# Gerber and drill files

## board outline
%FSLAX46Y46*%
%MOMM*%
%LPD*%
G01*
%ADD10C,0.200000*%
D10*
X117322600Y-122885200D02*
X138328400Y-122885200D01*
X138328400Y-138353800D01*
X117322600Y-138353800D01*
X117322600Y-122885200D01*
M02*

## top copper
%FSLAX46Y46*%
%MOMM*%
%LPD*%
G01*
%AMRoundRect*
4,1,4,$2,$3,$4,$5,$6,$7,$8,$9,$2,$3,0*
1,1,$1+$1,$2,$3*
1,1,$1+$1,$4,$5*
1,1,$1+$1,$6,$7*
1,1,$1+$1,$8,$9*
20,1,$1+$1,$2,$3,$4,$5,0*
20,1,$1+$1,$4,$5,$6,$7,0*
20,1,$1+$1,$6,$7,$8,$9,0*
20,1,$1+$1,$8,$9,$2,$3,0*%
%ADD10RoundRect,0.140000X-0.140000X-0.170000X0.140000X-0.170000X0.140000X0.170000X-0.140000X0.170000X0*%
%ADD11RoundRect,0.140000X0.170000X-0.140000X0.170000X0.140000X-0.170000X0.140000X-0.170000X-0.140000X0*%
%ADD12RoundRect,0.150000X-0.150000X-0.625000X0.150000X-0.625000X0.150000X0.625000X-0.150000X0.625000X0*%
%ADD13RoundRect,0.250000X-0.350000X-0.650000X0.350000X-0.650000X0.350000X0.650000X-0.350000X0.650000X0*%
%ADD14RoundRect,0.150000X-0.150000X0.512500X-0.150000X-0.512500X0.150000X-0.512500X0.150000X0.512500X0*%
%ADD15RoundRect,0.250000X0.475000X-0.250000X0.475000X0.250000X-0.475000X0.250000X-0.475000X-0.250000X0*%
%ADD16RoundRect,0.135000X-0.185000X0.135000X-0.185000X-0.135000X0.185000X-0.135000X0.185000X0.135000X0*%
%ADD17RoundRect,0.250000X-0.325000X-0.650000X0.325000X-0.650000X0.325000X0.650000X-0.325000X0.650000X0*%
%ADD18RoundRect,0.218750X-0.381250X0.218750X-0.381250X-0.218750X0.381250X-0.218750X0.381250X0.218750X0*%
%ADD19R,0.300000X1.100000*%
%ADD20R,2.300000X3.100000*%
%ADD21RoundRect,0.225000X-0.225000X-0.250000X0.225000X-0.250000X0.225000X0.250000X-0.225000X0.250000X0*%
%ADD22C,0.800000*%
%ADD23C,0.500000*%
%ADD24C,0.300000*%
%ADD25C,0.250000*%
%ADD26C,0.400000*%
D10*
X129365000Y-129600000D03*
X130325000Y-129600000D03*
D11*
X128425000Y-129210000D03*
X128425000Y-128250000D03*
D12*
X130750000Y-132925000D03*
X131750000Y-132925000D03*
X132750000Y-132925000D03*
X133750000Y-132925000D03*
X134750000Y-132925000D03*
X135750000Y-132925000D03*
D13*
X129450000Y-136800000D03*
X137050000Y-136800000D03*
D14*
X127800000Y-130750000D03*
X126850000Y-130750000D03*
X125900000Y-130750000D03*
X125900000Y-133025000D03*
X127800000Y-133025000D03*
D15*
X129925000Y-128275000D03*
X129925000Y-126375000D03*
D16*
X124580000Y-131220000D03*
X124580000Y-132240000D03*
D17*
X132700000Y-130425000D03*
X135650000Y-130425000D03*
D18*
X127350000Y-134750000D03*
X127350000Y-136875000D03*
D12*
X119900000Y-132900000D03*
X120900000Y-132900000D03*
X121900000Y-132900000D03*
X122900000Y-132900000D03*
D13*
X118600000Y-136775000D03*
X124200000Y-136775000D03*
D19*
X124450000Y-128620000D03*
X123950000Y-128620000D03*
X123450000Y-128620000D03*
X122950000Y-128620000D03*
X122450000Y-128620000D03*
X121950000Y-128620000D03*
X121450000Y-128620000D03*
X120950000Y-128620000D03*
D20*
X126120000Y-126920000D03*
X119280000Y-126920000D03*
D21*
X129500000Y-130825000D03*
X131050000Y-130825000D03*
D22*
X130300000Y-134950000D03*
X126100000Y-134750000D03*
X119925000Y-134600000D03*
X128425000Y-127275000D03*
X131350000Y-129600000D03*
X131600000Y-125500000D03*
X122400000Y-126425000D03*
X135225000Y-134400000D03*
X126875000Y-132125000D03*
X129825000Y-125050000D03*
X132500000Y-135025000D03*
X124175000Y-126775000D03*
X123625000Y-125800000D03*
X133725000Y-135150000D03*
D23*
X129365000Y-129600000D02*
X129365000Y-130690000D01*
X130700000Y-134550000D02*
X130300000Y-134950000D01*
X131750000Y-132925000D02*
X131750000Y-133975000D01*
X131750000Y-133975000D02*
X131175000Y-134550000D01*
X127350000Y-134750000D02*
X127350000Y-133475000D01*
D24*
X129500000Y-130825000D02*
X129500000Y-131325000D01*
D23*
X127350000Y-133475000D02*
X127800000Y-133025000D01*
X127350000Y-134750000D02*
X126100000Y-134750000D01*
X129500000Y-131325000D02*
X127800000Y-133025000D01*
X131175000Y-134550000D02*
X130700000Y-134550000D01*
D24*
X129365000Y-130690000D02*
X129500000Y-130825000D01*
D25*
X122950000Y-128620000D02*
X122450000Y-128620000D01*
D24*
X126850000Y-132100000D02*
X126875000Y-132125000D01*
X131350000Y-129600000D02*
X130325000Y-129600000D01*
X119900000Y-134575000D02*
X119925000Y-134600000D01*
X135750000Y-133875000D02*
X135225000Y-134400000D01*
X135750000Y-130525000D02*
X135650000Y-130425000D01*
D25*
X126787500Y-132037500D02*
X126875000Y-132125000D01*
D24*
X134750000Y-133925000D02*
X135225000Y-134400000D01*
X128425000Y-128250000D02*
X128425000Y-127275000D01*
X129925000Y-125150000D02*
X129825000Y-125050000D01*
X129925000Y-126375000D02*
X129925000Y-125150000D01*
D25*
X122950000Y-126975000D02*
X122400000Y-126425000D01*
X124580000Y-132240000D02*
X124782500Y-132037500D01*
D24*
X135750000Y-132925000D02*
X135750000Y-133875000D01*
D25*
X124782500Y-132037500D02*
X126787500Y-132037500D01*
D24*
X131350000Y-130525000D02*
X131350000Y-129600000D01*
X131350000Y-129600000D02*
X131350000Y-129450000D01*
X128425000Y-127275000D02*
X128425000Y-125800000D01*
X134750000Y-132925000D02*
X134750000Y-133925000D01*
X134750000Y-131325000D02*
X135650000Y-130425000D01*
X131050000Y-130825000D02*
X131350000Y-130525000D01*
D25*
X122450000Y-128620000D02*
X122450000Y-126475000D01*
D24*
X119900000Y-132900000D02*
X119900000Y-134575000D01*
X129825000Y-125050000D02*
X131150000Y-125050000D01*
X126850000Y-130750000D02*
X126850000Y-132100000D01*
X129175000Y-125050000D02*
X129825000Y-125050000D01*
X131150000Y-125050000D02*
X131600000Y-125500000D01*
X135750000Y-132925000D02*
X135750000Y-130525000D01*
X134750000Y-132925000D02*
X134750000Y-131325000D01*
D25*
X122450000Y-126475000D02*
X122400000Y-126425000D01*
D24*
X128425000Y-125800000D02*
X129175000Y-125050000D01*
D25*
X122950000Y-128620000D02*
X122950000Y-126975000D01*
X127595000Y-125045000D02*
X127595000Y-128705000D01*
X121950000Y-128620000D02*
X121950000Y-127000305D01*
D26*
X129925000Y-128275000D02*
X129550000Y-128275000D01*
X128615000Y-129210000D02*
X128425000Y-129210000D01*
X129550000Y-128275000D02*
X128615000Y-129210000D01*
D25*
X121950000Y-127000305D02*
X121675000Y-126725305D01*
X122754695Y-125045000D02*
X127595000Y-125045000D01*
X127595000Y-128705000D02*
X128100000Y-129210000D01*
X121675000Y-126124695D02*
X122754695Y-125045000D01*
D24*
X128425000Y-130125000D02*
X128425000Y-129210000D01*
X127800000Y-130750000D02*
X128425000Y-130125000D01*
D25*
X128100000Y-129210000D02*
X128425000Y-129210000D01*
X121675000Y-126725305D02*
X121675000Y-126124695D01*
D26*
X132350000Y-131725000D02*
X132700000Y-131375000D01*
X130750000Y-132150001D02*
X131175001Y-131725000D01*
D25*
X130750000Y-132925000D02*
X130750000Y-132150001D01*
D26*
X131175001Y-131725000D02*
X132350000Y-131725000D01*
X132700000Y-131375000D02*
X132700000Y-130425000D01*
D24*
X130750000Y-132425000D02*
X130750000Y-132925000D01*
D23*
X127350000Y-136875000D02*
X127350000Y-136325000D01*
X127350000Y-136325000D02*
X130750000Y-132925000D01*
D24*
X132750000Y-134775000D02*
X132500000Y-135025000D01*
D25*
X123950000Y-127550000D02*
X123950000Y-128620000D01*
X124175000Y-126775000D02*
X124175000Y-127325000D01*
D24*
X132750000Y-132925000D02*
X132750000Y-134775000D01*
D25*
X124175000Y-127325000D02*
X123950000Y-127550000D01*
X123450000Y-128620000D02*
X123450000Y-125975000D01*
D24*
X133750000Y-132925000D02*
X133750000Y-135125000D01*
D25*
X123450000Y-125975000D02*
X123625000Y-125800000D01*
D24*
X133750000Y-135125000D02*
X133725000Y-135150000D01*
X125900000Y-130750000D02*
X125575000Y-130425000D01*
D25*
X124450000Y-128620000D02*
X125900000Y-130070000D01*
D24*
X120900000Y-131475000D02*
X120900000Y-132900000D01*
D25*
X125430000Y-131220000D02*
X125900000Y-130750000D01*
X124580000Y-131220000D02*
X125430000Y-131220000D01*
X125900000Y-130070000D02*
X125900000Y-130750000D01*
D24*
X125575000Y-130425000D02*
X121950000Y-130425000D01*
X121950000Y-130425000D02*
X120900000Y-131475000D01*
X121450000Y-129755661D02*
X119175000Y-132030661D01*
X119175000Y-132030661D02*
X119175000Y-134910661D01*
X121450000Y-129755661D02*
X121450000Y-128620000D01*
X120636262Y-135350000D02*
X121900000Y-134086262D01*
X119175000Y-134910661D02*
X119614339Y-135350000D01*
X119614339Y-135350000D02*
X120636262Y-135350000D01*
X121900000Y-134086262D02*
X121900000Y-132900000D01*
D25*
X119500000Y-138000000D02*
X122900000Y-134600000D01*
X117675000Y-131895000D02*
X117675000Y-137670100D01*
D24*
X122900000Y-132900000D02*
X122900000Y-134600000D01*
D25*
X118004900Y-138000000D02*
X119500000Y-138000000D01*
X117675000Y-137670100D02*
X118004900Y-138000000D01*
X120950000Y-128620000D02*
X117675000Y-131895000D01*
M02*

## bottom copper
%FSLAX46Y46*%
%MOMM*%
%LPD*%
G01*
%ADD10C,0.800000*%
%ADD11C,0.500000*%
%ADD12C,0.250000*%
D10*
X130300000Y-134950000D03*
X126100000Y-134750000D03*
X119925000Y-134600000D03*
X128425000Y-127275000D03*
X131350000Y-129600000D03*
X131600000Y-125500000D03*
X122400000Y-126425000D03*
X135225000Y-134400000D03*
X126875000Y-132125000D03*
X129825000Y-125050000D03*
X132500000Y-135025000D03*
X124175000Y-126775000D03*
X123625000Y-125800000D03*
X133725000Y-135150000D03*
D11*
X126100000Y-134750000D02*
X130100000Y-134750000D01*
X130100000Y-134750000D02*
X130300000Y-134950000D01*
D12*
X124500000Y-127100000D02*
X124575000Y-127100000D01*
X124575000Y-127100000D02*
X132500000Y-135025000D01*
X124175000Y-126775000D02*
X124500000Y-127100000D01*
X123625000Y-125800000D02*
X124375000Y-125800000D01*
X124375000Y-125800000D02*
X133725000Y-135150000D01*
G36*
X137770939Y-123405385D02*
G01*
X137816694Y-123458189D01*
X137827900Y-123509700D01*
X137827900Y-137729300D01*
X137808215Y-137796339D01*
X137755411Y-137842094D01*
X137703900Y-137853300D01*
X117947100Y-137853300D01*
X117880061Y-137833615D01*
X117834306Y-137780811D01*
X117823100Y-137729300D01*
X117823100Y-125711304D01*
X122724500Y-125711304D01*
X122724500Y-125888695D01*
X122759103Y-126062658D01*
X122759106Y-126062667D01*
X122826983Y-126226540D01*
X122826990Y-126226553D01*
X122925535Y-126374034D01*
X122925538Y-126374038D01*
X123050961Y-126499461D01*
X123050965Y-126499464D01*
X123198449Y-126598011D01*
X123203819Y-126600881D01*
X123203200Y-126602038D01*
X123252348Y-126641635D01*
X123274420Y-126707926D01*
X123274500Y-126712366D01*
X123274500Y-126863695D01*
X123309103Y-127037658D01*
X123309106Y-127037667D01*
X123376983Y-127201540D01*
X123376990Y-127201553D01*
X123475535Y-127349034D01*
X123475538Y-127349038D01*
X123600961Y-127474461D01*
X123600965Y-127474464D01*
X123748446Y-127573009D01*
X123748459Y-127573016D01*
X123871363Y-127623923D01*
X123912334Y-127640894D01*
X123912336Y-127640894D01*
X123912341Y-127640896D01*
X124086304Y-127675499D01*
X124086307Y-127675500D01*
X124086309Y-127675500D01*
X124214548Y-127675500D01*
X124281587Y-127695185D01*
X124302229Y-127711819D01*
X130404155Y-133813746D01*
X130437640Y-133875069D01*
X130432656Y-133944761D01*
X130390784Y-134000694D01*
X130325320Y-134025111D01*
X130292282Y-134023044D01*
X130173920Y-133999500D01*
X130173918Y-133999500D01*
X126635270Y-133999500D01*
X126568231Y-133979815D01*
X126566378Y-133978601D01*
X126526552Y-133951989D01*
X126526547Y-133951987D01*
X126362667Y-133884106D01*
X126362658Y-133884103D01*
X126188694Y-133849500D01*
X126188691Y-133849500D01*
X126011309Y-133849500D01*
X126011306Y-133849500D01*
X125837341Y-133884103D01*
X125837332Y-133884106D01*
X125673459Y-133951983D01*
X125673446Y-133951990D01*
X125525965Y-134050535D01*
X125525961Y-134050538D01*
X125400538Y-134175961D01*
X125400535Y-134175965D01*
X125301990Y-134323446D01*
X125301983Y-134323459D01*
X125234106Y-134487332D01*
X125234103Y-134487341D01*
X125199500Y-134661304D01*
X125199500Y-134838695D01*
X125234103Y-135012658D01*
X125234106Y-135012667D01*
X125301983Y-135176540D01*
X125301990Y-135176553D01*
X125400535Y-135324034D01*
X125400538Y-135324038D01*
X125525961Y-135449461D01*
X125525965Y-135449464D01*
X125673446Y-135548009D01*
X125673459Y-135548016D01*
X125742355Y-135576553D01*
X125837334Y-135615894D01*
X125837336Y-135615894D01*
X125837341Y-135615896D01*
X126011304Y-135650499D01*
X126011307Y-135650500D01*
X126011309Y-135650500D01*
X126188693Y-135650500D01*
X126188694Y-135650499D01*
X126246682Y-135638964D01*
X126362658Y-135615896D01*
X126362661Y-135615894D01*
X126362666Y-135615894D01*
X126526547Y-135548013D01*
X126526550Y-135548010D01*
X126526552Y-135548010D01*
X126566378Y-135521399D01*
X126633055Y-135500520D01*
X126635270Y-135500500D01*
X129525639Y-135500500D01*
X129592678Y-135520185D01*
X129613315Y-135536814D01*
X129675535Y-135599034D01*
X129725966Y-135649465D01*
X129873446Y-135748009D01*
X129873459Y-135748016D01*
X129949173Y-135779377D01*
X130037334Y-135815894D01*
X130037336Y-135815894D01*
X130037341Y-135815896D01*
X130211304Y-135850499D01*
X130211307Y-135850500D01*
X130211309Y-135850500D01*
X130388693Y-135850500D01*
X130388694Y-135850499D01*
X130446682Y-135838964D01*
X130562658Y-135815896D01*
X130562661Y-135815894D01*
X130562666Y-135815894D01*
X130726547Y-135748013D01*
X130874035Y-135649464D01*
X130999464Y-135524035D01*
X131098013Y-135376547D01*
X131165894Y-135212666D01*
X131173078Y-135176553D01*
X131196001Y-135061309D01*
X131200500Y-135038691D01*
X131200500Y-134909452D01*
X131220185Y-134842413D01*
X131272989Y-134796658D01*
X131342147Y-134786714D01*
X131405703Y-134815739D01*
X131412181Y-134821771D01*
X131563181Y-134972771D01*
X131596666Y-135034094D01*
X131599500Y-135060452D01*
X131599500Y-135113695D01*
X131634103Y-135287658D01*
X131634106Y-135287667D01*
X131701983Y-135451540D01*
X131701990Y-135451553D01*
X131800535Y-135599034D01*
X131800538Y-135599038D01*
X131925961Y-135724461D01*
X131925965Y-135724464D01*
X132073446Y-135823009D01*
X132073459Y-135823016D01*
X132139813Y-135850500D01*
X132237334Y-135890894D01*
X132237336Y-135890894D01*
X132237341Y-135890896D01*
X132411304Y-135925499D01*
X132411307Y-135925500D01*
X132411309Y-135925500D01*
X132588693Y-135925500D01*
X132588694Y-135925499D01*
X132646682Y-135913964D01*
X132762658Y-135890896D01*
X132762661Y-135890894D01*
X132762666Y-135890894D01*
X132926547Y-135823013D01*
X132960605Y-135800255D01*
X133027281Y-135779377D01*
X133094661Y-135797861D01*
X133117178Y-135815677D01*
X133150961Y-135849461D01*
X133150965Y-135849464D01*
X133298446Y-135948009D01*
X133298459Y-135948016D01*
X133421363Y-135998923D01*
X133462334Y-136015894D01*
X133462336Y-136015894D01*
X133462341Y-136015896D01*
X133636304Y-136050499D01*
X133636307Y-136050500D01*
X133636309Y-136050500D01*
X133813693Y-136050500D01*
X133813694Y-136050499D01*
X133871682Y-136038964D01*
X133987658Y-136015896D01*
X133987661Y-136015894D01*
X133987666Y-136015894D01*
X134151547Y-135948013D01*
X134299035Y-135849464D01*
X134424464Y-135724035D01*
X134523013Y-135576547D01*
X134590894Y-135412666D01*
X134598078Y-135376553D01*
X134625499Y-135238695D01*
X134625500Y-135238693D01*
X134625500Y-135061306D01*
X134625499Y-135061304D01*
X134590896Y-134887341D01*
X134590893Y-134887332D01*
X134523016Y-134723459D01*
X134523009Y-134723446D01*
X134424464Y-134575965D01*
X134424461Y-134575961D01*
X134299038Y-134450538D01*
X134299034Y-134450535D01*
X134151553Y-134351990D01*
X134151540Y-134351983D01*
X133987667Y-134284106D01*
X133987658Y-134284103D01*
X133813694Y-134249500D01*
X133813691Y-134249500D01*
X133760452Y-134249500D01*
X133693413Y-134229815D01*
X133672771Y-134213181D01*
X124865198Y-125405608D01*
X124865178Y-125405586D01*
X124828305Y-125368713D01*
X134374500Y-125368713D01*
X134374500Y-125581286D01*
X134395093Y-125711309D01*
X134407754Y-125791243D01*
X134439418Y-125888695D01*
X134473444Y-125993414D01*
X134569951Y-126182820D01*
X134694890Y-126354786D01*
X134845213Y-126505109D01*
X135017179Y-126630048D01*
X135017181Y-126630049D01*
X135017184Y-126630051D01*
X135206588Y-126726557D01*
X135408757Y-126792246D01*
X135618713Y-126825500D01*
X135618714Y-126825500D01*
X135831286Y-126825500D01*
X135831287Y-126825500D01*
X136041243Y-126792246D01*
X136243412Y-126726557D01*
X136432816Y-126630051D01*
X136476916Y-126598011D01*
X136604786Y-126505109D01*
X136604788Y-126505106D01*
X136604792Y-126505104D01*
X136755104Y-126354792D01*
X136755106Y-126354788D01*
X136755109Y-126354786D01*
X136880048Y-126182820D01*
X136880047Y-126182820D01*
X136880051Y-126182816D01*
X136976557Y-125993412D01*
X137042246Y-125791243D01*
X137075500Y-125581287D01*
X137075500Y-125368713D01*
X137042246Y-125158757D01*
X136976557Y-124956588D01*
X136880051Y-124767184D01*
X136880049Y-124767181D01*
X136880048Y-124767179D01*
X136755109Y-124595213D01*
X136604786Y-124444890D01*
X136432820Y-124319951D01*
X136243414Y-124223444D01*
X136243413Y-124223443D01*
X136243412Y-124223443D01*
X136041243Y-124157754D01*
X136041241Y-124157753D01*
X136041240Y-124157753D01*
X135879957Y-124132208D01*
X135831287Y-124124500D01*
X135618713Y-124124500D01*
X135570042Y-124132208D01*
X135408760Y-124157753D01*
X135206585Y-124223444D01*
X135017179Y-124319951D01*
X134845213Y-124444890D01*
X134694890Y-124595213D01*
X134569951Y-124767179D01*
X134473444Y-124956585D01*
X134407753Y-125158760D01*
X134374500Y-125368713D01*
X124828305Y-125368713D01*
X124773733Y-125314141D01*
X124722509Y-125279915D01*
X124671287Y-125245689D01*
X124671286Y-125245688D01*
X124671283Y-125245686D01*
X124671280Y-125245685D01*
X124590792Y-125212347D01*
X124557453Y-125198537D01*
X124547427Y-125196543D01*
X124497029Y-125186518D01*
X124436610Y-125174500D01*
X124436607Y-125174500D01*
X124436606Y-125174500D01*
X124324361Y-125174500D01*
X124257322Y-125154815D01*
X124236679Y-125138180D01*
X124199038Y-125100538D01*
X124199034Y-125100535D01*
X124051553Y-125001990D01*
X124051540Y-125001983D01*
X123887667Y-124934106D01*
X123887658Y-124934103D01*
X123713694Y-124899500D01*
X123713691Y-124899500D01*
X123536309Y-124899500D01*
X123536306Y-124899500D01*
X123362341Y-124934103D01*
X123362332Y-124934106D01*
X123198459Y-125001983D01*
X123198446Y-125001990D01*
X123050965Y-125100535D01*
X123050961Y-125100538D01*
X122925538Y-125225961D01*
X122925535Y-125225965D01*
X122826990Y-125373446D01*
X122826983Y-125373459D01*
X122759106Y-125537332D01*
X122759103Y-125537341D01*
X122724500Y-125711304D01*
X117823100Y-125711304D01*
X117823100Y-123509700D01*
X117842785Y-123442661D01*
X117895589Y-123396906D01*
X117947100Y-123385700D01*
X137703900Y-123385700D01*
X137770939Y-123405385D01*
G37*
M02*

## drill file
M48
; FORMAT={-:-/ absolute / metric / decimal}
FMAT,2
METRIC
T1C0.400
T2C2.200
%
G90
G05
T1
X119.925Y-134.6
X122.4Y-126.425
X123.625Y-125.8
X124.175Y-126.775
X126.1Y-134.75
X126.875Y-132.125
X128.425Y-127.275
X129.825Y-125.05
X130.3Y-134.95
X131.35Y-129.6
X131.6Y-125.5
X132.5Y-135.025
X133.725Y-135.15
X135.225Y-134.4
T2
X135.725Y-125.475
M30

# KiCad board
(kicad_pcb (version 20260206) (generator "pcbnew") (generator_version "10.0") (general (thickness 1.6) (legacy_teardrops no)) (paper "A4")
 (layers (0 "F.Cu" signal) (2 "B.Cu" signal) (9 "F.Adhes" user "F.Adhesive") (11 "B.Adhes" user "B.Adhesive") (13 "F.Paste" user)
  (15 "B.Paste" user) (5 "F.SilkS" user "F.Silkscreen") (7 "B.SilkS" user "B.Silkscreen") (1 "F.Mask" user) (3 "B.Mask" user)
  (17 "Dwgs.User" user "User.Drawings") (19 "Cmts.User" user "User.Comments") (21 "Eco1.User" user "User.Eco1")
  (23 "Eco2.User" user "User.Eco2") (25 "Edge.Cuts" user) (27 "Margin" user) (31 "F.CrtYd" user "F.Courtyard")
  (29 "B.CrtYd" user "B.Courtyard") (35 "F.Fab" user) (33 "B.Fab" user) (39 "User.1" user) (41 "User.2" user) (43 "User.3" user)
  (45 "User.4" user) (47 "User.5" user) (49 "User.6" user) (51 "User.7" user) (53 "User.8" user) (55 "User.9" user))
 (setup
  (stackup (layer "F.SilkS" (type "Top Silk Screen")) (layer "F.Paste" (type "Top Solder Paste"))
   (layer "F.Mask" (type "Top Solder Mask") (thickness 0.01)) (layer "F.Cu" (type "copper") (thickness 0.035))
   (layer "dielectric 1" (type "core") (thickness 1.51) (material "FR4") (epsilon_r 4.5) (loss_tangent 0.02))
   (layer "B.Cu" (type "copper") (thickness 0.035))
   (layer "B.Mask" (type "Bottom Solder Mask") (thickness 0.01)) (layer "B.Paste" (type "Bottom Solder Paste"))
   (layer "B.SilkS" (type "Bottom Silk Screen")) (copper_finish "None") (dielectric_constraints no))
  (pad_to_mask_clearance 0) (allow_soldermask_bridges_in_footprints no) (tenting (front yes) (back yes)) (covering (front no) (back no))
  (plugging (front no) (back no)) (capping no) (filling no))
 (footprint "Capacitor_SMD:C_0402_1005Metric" (layer "F.Cu") (at 129.845 129.6)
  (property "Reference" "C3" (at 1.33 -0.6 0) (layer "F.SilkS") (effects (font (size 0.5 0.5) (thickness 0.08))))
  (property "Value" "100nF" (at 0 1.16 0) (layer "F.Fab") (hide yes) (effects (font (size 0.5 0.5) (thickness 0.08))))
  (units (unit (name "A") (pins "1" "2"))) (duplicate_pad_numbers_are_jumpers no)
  (pad "1" smd roundrect (at -0.48 0) (size 0.56 0.62) (layers "F.Cu" "F.Mask" "F.Paste") (roundrect_rratio 0.25) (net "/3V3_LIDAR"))
  (pad "2" smd roundrect (at 0.48 0) (size 0.56 0.62) (layers "F.Cu" "F.Mask" "F.Paste") (roundrect_rratio 0.25) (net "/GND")))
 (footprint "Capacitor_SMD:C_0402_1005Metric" (layer "F.Cu") (at 128.425 128.73 90)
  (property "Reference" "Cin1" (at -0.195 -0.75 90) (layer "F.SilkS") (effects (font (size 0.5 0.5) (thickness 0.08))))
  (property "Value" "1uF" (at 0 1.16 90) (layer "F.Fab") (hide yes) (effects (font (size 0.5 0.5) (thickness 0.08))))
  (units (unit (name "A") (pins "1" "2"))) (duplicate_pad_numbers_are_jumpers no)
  (pad "1" smd roundrect (at -0.48 0 90) (size 0.56 0.62) (layers "F.Cu" "F.Mask" "F.Paste") (roundrect_rratio 0.25) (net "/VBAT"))
  (pad "2" smd roundrect (at 0.48 0 90) (size 0.56 0.62) (layers "F.Cu" "F.Mask" "F.Paste") (roundrect_rratio 0.25) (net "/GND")))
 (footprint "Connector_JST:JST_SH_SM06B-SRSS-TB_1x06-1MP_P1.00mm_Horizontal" (layer "F.Cu") (at 133.25 134.925)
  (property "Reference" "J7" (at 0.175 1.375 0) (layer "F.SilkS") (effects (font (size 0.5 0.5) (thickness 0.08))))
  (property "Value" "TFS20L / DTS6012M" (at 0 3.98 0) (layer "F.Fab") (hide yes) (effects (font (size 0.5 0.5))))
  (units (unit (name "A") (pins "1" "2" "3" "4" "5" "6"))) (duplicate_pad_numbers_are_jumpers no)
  (pad "1" smd roundrect (at -2.5 -2) (size 0.6 1.55) (layers "F.Cu" "F.Mask" "F.Paste") (roundrect_rratio 0.25) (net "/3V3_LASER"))
  (pad "2" smd roundrect (at -1.5 -2) (size 0.6 1.55) (layers "F.Cu" "F.Mask" "F.Paste") (roundrect_rratio 0.25) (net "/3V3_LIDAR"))
  (pad "3" smd roundrect (at -0.5 -2) (size 0.6 1.55) (layers "F.Cu" "F.Mask" "F.Paste") (roundrect_rratio 0.25) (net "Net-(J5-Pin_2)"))
  (pad "4" smd roundrect (at 0.5 -2) (size 0.6 1.55) (layers "F.Cu" "F.Mask" "F.Paste") (roundrect_rratio 0.25) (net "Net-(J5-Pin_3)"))
  (pad "5" smd roundrect (at 1.5 -2) (size 0.6 1.55) (layers "F.Cu" "F.Mask" "F.Paste") (roundrect_rratio 0.25) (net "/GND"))
  (pad "6" smd roundrect (at 2.5 -2) (size 0.6 1.55) (layers "F.Cu" "F.Mask" "F.Paste") (roundrect_rratio 0.25) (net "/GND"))
  (pad "MP" smd roundrect (at -3.8 1.875) (size 1.2 1.8) (layers "F.Cu" "F.Mask" "F.Paste") (roundrect_rratio 0.208333))
  (pad "MP" smd roundrect (at 3.8 1.875) (size 1.2 1.8) (layers "F.Cu" "F.Mask" "F.Paste") (roundrect_rratio 0.208333)))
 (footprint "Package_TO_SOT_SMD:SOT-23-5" (layer "F.Cu") (at 126.85 131.8875 -90)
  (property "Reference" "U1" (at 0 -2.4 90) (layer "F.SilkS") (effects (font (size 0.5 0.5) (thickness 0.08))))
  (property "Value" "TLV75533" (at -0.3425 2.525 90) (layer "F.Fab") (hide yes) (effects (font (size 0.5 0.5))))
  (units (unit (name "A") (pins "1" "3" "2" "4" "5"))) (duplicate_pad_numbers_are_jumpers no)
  (pad "1" smd roundrect (at -1.1375 -0.95 270) (size 1.325 0.6) (layers "F.Cu" "F.Mask" "F.Paste") (roundrect_rratio 0.25) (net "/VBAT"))
  (pad "2" smd roundrect (at -1.1375 0 270) (size 1.325 0.6) (layers "F.Cu" "F.Mask" "F.Paste") (roundrect_rratio 0.25) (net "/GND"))
  (pad "3" smd roundrect (at -1.1375 0.95 270) (size 1.325 0.6) (layers "F.Cu" "F.Mask" "F.Paste") (roundrect_rratio 0.25) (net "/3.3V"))
  (pad "4" smd roundrect (at 1.1375 0.95 270) (size 1.325 0.6) (layers "F.Cu" "F.Mask" "F.Paste") (roundrect_rratio 0.25)
   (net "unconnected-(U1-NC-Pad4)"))
  (pad "5" smd roundrect (at 1.1375 -0.95 270) (size 1.325 0.6) (layers "F.Cu" "F.Mask" "F.Paste") (roundrect_rratio 0.25)
   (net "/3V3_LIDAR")))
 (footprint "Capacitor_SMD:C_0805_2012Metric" (layer "F.Cu") (at 129.925 127.325 90)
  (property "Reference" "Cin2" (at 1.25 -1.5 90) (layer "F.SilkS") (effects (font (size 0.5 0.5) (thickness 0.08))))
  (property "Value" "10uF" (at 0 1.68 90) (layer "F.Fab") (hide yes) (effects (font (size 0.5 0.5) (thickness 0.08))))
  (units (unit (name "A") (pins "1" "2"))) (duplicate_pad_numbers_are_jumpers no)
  (pad "1" smd roundrect (at -0.95 0 90) (size 1 1.45) (layers "F.Cu" "F.Mask" "F.Paste") (roundrect_rratio 0.25) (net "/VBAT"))
  (pad "2" smd roundrect (at 0.95 0 90) (size 1 1.45) (layers "F.Cu" "F.Mask" "F.Paste") (roundrect_rratio 0.25) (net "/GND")))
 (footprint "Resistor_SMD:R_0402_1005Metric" (layer "F.Cu") (at 124.58 131.73 -90)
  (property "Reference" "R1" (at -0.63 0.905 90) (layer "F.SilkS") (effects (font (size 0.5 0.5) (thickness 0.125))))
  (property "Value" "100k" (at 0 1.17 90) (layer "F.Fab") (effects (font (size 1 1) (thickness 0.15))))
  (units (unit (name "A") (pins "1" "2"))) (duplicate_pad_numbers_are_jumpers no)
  (pad "1" smd roundrect (at -0.51 0 270) (size 0.54 0.64) (layers "F.Cu" "F.Mask" "F.Paste") (roundrect_rratio 0.25) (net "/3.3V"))
  (pad "2" smd roundrect (at 0.51 0 270) (size 0.54 0.64) (layers "F.Cu" "F.Mask" "F.Paste") (roundrect_rratio 0.25) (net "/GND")))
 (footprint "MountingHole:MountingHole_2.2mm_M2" (layer "F.Cu") (at 135.725 125.475)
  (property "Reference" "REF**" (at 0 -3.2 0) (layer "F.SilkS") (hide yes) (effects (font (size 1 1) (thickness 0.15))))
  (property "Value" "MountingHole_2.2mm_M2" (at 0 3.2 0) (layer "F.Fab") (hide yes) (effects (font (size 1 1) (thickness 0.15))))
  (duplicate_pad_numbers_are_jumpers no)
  (pad "" np_thru_hole circle (at 0 0) (size 2.2 2.2) (drill 2.2) (layers "*.Cu" "*.Mask")))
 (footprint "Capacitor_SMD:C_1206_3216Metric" (layer "F.Cu") (at 134.175 130.425)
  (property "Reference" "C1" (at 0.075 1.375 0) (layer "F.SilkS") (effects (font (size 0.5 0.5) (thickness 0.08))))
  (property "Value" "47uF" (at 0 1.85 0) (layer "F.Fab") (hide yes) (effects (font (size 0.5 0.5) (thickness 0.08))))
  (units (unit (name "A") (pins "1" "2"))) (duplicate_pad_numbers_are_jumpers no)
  (pad "1" smd roundrect (at -1.475 0) (size 1.15 1.8) (layers "F.Cu" "F.Mask" "F.Paste") (roundrect_rratio 0.217391) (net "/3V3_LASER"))
  (pad "2" smd roundrect (at 1.475 0) (size 1.15 1.8) (layers "F.Cu" "F.Mask" "F.Paste") (roundrect_rratio 0.217391) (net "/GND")))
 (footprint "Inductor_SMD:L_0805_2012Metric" (layer "F.Cu") (at 127.35 135.8125 -90)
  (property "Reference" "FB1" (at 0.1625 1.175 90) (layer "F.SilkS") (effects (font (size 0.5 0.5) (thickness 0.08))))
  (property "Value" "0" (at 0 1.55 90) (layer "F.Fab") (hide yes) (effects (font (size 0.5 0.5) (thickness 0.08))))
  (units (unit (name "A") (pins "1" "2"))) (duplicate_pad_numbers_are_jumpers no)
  (pad "1" smd roundrect (at -1.0625 0 270) (size 0.875 1.2) (layers "F.Cu" "F.Mask" "F.Paste") (roundrect_rratio 0.25) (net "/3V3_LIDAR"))
  (pad "2" smd roundrect (at 1.0625 0 270) (size 0.875 1.2) (layers "F.Cu" "F.Mask" "F.Paste") (roundrect_rratio 0.25) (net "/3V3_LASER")))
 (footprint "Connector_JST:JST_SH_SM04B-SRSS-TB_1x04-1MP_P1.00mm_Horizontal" (layer "F.Cu") (at 121.4 134.9)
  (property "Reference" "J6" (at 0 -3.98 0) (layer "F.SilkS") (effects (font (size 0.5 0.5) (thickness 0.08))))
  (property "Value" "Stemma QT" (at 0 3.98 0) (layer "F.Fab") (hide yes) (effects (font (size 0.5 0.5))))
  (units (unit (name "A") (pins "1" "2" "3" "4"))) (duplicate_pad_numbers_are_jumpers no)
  (pad "1" smd roundrect (at -1.5 -2) (size 0.6 1.55) (layers "F.Cu" "F.Mask" "F.Paste") (roundrect_rratio 0.25) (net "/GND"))
  (pad "2" smd roundrect (at -0.5 -2) (size 0.6 1.55) (layers "F.Cu" "F.Mask" "F.Paste") (roundrect_rratio 0.25) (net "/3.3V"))
  (pad "3" smd roundrect (at 0.5 -2) (size 0.6 1.55) (layers "F.Cu" "F.Mask" "F.Paste") (roundrect_rratio 0.25) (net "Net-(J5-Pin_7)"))
  (pad "4" smd roundrect (at 1.5 -2) (size 0.6 1.55) (layers "F.Cu" "F.Mask" "F.Paste") (roundrect_rratio 0.25) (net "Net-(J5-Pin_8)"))
  (pad "MP" smd roundrect (at -2.8 1.875) (size 1.2 1.8) (layers "F.Cu" "F.Mask" "F.Paste") (roundrect_rratio 0.208333))
  (pad "MP" smd roundrect (at 2.8 1.875) (size 1.2 1.8) (layers "F.Cu" "F.Mask" "F.Paste") (roundrect_rratio 0.208333)))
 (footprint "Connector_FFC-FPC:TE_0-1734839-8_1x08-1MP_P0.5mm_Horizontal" (layer "F.Cu") (at 122.7 127.27 180)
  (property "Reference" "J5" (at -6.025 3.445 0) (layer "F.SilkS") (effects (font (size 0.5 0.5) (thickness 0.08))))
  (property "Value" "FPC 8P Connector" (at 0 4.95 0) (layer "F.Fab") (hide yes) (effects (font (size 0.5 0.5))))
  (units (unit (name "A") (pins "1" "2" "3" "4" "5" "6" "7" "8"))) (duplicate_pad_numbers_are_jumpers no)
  (pad "1" smd rect (at -1.75 -1.35 180) (size 0.3 1.1) (layers "F.Cu" "F.Mask" "F.Paste") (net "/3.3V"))
  (pad "2" smd rect (at -1.25 -1.35 180) (size 0.3 1.1) (layers "F.Cu" "F.Mask" "F.Paste") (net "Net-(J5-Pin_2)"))
  (pad "3" smd rect (at -0.75 -1.35 180) (size 0.3 1.1) (layers "F.Cu" "F.Mask" "F.Paste") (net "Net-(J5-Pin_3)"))
  (pad "4" smd rect (at -0.25 -1.35 180) (size 0.3 1.1) (layers "F.Cu" "F.Mask" "F.Paste") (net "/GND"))
  (pad "5" smd rect (at 0.25 -1.35 180) (size 0.3 1.1) (layers "F.Cu" "F.Mask" "F.Paste") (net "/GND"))
  (pad "6" smd rect (at 0.75 -1.35 180) (size 0.3 1.1) (layers "F.Cu" "F.Mask" "F.Paste") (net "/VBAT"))
  (pad "7" smd rect (at 1.25 -1.35 180) (size 0.3 1.1) (layers "F.Cu" "F.Mask" "F.Paste") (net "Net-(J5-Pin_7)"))
  (pad "8" smd rect (at 1.75 -1.35 180) (size 0.3 1.1) (layers "F.Cu" "F.Mask" "F.Paste") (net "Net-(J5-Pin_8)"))
  (pad "MP" smd rect (at -3.42 0.35 180) (size 2.3 3.1) (layers "F.Cu" "F.Mask" "F.Paste"))
  (pad "MP" smd rect (at 3.42 0.35 180) (size 2.3 3.1) (layers "F.Cu" "F.Mask" "F.Paste")))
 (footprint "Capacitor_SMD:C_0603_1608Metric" (layer "F.Cu") (at 130.275 130.825)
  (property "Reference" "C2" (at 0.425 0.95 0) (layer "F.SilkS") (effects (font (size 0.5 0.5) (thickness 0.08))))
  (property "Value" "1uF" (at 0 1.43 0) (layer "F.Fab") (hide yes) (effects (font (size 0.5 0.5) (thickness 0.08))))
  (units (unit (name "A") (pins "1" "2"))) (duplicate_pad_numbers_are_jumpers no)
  (pad "1" smd roundrect (at -0.775 0) (size 0.9 0.95) (layers "F.Cu" "F.Mask" "F.Paste") (roundrect_rratio 0.25) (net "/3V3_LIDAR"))
  (pad "2" smd roundrect (at 0.775 0) (size 0.9 0.95) (layers "F.Cu" "F.Mask" "F.Paste") (roundrect_rratio 0.25) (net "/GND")))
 (gr_rect (start 117.3226 122.8852) (end 138.3284 138.3538) (stroke (width 0.2) (type default)) (fill no) (layer "Edge.Cuts"))
 (segment (start 129.365 129.6) (end 129.365 130.69) (width 0.5) (layer "F.Cu") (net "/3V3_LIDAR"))
 (segment (start 130.7 134.55) (end 130.3 134.95) (width 0.5) (layer "F.Cu") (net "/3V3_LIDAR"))
 (segment (start 131.75 132.925) (end 131.75 133.975) (width 0.5) (layer "F.Cu") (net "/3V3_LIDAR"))
 (segment (start 131.75 133.975) (end 131.175 134.55) (width 0.5) (layer "F.Cu") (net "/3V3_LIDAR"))
 (segment (start 127.35 134.75) (end 127.35 133.475) (width 0.5) (layer "F.Cu") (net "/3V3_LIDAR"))
 (segment (start 129.5 130.825) (end 129.5 131.325) (width 0.3) (layer "F.Cu") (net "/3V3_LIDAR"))
 (segment (start 127.35 133.475) (end 127.8 133.025) (width 0.5) (layer "F.Cu") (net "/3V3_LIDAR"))
 (segment (start 127.35 134.75) (end 126.1 134.75) (width 0.5) (layer "F.Cu") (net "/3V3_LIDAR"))
 (segment (start 129.5 131.325) (end 127.8 133.025) (width 0.5) (layer "F.Cu") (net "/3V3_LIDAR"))
 (segment (start 131.175 134.55) (end 130.7 134.55) (width 0.5) (layer "F.Cu") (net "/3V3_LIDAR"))
 (segment (start 129.365 130.69) (end 129.5 130.825) (width 0.3) (layer "F.Cu") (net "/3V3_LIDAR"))
 (via (at 130.3 134.95) (size 0.8) (drill 0.4) (layers "F.Cu" "B.Cu") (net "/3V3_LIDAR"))
 (via (at 126.1 134.75) (size 0.8) (drill 0.4) (layers "F.Cu" "B.Cu") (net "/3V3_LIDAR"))
 (segment (start 126.1 134.75) (end 130.1 134.75) (width 0.5) (layer "B.Cu") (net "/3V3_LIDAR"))
 (segment (start 130.1 134.75) (end 130.3 134.95) (width 0.5) (layer "B.Cu") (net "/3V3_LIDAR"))
 (segment (start 122.95 128.62) (end 122.45 128.62) (width 0.25) (layer "F.Cu") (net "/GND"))
 (segment (start 126.85 132.1) (end 126.875 132.125) (width 0.3) (layer "F.Cu") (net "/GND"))
 (segment (start 131.35 129.6) (end 130.325 129.6) (width 0.3) (layer "F.Cu") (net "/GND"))
 (segment (start 119.9 134.575) (end 119.925 134.6) (width 0.3) (layer "F.Cu") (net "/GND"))
 (segment (start 135.75 133.875) (end 135.225 134.4) (width 0.3) (layer "F.Cu") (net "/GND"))
 (segment (start 135.75 130.525) (end 135.65 130.425) (width 0.3) (layer "F.Cu") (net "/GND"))
 (segment (start 126.7875 132.0375) (end 126.875 132.125) (width 0.25) (layer "F.Cu") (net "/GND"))
 (segment (start 134.75 133.925) (end 135.225 134.4) (width 0.3) (layer "F.Cu") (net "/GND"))
 (segment (start 128.425 128.25) (end 128.425 127.275) (width 0.3) (layer "F.Cu") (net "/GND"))
 (segment (start 129.925 125.15) (end 129.825 125.05) (width 0.3) (layer "F.Cu") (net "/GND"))
 (segment (start 129.925 126.375) (end 129.925 125.15) (width 0.3) (layer "F.Cu") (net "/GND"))
 (segment (start 122.95 126.975) (end 122.4 126.425) (width 0.25) (layer "F.Cu") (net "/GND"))
 (segment (start 124.58 132.24) (end 124.7825 132.0375) (width 0.25) (layer "F.Cu") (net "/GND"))
 (segment (start 135.75 132.925) (end 135.75 133.875) (width 0.3) (layer "F.Cu") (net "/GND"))
 (segment (start 124.7825 132.0375) (end 126.7875 132.0375) (width 0.25) (layer "F.Cu") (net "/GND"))
 (segment (start 131.35 130.525) (end 131.35 129.6) (width 0.3) (layer "F.Cu") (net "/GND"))
 (segment (start 131.35 129.6) (end 131.35 129.45) (width 0.3) (layer "F.Cu") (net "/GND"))
 (segment (start 128.425 127.275) (end 128.425 125.8) (width 0.3) (layer "F.Cu") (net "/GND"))
 (segment (start 134.75 132.925) (end 134.75 133.925) (width 0.3) (layer "F.Cu") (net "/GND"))
 (segment (start 134.75 131.325) (end 135.65 130.425) (width 0.3) (layer "F.Cu") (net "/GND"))
 (segment (start 131.05 130.825) (end 131.35 130.525) (width 0.3) (layer "F.Cu") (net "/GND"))
 (segment (start 122.45 128.62) (end 122.45 126.475) (width 0.25) (layer "F.Cu") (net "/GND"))
 (segment (start 119.9 132.9) (end 119.9 134.575) (width 0.3) (layer "F.Cu") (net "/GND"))
 (segment (start 129.825 125.05) (end 131.15 125.05) (width 0.3) (layer "F.Cu") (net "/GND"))
 (segment (start 126.85 130.75) (end 126.85 132.1) (width 0.3) (layer "F.Cu") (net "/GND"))
 (segment (start 129.175 125.05) (end 129.825 125.05) (width 0.3) (layer "F.Cu") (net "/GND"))
 (segment (start 131.15 125.05) (end 131.6 125.5) (width 0.3) (layer "F.Cu") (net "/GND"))
 (segment (start 135.75 132.925) (end 135.75 130.525) (width 0.3) (layer "F.Cu") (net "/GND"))
 (segment (start 134.75 132.925) (end 134.75 131.325) (width 0.3) (layer "F.Cu") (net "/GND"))
 (segment (start 122.45 126.475) (end 122.4 126.425) (width 0.25) (layer "F.Cu") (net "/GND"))
 (segment (start 128.425 125.8) (end 129.175 125.05) (width 0.3) (layer "F.Cu") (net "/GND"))
 (segment (start 122.95 128.62) (end 122.95 126.975) (width 0.25) (layer "F.Cu") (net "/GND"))
 (via (at 119.925 134.6) (size 0.8) (drill 0.4) (layers "F.Cu" "B.Cu") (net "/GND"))
 (via (at 128.425 127.275) (size 0.8) (drill 0.4) (layers "F.Cu" "B.Cu") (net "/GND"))
 (via (at 131.35 129.6) (size 0.8) (drill 0.4) (layers "F.Cu" "B.Cu") (free yes) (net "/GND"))
 (via (at 131.6 125.5) (size 0.8) (drill 0.4) (layers "F.Cu" "B.Cu") (free yes) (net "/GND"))
 (via (at 122.4 126.425) (size 0.8) (drill 0.4) (layers "F.Cu" "B.Cu") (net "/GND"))
 (via (at 135.225 134.4) (size 0.8) (drill 0.4) (layers "F.Cu" "B.Cu") (free yes) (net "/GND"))
 (via (at 126.875 132.125) (size 0.8) (drill 0.4) (layers "F.Cu" "B.Cu") (free yes) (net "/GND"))
 (via (at 129.825 125.05) (size 0.8) (drill 0.4) (layers "F.Cu" "B.Cu") (free yes) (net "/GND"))
 (segment (start 127.595 125.045) (end 127.595 128.705) (width 0.25) (layer "F.Cu") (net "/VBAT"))
 (segment (start 121.95 128.62) (end 121.95 127.000305) (width 0.25) (layer "F.Cu") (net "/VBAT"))
 (segment (start 129.925 128.275) (end 129.55 128.275) (width 0.4) (layer "F.Cu") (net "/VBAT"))
 (segment (start 128.615 129.21) (end 128.425 129.21) (width 0.4) (layer "F.Cu") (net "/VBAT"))
 (segment (start 129.55 128.275) (end 128.615 129.21) (width 0.4) (layer "F.Cu") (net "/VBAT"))
 (segment (start 121.95 127.000305) (end 121.675 126.725305) (width 0.25) (layer "F.Cu") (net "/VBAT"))
 (segment (start 122.754695 125.045) (end 127.595 125.045) (width 0.25) (layer "F.Cu") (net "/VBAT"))
 (segment (start 127.595 128.705) (end 128.1 129.21) (width 0.25) (layer "F.Cu") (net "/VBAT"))
 (segment (start 121.675 126.124695) (end 122.754695 125.045) (width 0.25) (layer "F.Cu") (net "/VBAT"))
 (segment (start 128.425 130.125) (end 128.425 129.21) (width 0.3) (layer "F.Cu") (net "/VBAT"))
 (segment (start 127.8 130.75) (end 128.425 130.125) (width 0.3) (layer "F.Cu") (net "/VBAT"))
 (segment (start 128.1 129.21) (end 128.425 129.21) (width 0.25) (layer "F.Cu") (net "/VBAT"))
 (segment (start 121.675 126.725305) (end 121.675 126.124695) (width 0.25) (layer "F.Cu") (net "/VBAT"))
 (segment (start 132.35 131.725) (end 132.7 131.375) (width 0.4) (layer "F.Cu") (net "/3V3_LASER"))
 (segment (start 130.75 132.150001) (end 131.175001 131.725) (width 0.4) (layer "F.Cu") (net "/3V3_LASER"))
 (segment (start 130.75 132.925) (end 130.75 132.150001) (width 0.25) (layer "F.Cu") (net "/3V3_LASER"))
 (segment (start 131.175001 131.725) (end 132.35 131.725) (width 0.4) (layer "F.Cu") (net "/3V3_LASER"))
 (segment (start 132.7 131.375) (end 132.7 130.425) (width 0.4) (layer "F.Cu") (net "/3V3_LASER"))
 (segment (start 130.75 132.425) (end 130.75 132.925) (width 0.3) (layer "F.Cu") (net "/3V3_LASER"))
 (segment (start 127.35 136.875) (end 127.35 136.325) (width 0.5) (layer "F.Cu") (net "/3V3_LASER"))
 (segment (start 127.35 136.325) (end 130.75 132.925) (width 0.5) (layer "F.Cu") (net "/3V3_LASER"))
 (segment (start 132.75 134.775) (end 132.5 135.025) (width 0.3) (layer "F.Cu") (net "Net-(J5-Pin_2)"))
 (segment (start 123.95 127.55) (end 123.95 128.62) (width 0.25) (layer "F.Cu") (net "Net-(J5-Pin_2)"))
 (segment (start 124.175 126.775) (end 124.175 127.325) (width 0.25) (layer "F.Cu") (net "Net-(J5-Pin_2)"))
 (segment (start 132.75 132.925) (end 132.75 134.775) (width 0.3) (layer "F.Cu") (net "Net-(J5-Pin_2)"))
 (segment (start 124.175 127.325) (end 123.95 127.55) (width 0.25) (layer "F.Cu") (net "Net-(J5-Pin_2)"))
 (via (at 132.5 135.025) (size 0.8) (drill 0.4) (layers "F.Cu" "B.Cu") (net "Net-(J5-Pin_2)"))
 (via (at 124.175 126.775) (size 0.8) (drill 0.4) (layers "F.Cu" "B.Cu") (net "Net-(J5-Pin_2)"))
 (segment (start 124.5 127.1) (end 124.575 127.1) (width 0.25) (layer "B.Cu") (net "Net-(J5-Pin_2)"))
 (segment (start 124.575 127.1) (end 132.5 135.025) (width 0.25) (layer "B.Cu") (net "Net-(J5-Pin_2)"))
 (segment (start 124.175 126.775) (end 124.5 127.1) (width 0.25) (layer "B.Cu") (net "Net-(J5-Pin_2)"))
 (segment (start 123.45 128.62) (end 123.45 125.975) (width 0.25) (layer "F.Cu") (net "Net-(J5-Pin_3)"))
 (segment (start 133.75 132.925) (end 133.75 135.125) (width 0.3) (layer "F.Cu") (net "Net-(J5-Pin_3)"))
 (segment (start 123.45 125.975) (end 123.625 125.8) (width 0.25) (layer "F.Cu") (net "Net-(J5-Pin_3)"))
 (segment (start 133.75 135.125) (end 133.725 135.15) (width 0.3) (layer "F.Cu") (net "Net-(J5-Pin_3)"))
 (via (at 123.625 125.8) (size 0.8) (drill 0.4) (layers "F.Cu" "B.Cu") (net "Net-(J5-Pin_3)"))
 (via (at 133.725 135.15) (size 0.8) (drill 0.4) (layers "F.Cu" "B.Cu") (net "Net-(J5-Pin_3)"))
 (segment (start 123.625 125.8) (end 124.375 125.8) (width 0.25) (layer "B.Cu") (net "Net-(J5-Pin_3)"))
 (segment (start 124.375 125.8) (end 133.725 135.15) (width 0.25) (layer "B.Cu") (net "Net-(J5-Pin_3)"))
 (segment (start 125.9 130.75) (end 125.575 130.425) (width 0.3) (layer "F.Cu") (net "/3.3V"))
 (segment (start 124.45 128.62) (end 125.9 130.07) (width 0.25) (layer "F.Cu") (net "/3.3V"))
 (segment (start 120.9 131.475) (end 120.9 132.9) (width 0.3) (layer "F.Cu") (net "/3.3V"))
 (segment (start 125.43 131.22) (end 125.9 130.75) (width 0.25) (layer "F.Cu") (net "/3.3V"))
 (segment (start 124.58 131.22) (end 125.43 131.22) (width 0.25) (layer "F.Cu") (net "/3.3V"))
 (segment (start 125.9 130.07) (end 125.9 130.75) (width 0.25) (layer "F.Cu") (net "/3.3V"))
 (segment (start 125.575 130.425) (end 121.95 130.425) (width 0.3) (layer "F.Cu") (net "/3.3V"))
 (segment (start 121.95 130.425) (end 120.9 131.475) (width 0.3) (layer "F.Cu") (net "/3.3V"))
 (segment (start 121.45 129.755661) (end 119.175 132.030661) (width 0.3) (layer "F.Cu") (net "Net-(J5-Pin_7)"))
 (segment (start 119.175 132.030661) (end 119.175 134.910661) (width 0.3) (layer "F.Cu") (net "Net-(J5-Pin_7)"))
 (segment (start 121.45 129.755661) (end 121.45 128.62) (width 0.3) (layer "F.Cu") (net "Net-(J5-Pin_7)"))
 (segment (start 120.636262 135.35) (end 121.9 134.086262) (width 0.3) (layer "F.Cu") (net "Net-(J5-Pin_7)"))
 (segment (start 119.175 134.910661) (end 119.614339 135.35) (width 0.3) (layer "F.Cu") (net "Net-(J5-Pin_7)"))
 (segment (start 119.614339 135.35) (end 120.636262 135.35) (width 0.3) (layer "F.Cu") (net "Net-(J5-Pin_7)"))
 (segment (start 121.9 134.086262) (end 121.9 132.9) (width 0.3) (layer "F.Cu") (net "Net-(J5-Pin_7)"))
 (segment (start 119.5 138) (end 122.9 134.6) (width 0.25) (layer "F.Cu") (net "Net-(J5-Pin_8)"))
 (segment (start 117.675 131.895) (end 117.675 137.6701) (width 0.25) (layer "F.Cu") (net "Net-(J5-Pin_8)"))
 (segment (start 122.9 132.9) (end 122.9 134.6) (width 0.3) (layer "F.Cu") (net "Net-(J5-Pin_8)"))
 (segment (start 118.0049 138) (end 119.5 138) (width 0.25) (layer "F.Cu") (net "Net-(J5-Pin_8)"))
 (segment (start 117.675 137.6701) (end 118.0049 138) (width 0.25) (layer "F.Cu") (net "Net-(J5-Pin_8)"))
 (segment (start 120.95 128.62) (end 117.675 131.895) (width 0.25) (layer "F.Cu") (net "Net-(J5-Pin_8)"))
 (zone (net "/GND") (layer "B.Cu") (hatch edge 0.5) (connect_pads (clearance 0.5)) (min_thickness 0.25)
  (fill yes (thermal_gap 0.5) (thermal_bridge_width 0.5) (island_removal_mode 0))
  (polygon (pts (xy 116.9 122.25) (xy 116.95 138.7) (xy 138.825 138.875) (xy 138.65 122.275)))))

